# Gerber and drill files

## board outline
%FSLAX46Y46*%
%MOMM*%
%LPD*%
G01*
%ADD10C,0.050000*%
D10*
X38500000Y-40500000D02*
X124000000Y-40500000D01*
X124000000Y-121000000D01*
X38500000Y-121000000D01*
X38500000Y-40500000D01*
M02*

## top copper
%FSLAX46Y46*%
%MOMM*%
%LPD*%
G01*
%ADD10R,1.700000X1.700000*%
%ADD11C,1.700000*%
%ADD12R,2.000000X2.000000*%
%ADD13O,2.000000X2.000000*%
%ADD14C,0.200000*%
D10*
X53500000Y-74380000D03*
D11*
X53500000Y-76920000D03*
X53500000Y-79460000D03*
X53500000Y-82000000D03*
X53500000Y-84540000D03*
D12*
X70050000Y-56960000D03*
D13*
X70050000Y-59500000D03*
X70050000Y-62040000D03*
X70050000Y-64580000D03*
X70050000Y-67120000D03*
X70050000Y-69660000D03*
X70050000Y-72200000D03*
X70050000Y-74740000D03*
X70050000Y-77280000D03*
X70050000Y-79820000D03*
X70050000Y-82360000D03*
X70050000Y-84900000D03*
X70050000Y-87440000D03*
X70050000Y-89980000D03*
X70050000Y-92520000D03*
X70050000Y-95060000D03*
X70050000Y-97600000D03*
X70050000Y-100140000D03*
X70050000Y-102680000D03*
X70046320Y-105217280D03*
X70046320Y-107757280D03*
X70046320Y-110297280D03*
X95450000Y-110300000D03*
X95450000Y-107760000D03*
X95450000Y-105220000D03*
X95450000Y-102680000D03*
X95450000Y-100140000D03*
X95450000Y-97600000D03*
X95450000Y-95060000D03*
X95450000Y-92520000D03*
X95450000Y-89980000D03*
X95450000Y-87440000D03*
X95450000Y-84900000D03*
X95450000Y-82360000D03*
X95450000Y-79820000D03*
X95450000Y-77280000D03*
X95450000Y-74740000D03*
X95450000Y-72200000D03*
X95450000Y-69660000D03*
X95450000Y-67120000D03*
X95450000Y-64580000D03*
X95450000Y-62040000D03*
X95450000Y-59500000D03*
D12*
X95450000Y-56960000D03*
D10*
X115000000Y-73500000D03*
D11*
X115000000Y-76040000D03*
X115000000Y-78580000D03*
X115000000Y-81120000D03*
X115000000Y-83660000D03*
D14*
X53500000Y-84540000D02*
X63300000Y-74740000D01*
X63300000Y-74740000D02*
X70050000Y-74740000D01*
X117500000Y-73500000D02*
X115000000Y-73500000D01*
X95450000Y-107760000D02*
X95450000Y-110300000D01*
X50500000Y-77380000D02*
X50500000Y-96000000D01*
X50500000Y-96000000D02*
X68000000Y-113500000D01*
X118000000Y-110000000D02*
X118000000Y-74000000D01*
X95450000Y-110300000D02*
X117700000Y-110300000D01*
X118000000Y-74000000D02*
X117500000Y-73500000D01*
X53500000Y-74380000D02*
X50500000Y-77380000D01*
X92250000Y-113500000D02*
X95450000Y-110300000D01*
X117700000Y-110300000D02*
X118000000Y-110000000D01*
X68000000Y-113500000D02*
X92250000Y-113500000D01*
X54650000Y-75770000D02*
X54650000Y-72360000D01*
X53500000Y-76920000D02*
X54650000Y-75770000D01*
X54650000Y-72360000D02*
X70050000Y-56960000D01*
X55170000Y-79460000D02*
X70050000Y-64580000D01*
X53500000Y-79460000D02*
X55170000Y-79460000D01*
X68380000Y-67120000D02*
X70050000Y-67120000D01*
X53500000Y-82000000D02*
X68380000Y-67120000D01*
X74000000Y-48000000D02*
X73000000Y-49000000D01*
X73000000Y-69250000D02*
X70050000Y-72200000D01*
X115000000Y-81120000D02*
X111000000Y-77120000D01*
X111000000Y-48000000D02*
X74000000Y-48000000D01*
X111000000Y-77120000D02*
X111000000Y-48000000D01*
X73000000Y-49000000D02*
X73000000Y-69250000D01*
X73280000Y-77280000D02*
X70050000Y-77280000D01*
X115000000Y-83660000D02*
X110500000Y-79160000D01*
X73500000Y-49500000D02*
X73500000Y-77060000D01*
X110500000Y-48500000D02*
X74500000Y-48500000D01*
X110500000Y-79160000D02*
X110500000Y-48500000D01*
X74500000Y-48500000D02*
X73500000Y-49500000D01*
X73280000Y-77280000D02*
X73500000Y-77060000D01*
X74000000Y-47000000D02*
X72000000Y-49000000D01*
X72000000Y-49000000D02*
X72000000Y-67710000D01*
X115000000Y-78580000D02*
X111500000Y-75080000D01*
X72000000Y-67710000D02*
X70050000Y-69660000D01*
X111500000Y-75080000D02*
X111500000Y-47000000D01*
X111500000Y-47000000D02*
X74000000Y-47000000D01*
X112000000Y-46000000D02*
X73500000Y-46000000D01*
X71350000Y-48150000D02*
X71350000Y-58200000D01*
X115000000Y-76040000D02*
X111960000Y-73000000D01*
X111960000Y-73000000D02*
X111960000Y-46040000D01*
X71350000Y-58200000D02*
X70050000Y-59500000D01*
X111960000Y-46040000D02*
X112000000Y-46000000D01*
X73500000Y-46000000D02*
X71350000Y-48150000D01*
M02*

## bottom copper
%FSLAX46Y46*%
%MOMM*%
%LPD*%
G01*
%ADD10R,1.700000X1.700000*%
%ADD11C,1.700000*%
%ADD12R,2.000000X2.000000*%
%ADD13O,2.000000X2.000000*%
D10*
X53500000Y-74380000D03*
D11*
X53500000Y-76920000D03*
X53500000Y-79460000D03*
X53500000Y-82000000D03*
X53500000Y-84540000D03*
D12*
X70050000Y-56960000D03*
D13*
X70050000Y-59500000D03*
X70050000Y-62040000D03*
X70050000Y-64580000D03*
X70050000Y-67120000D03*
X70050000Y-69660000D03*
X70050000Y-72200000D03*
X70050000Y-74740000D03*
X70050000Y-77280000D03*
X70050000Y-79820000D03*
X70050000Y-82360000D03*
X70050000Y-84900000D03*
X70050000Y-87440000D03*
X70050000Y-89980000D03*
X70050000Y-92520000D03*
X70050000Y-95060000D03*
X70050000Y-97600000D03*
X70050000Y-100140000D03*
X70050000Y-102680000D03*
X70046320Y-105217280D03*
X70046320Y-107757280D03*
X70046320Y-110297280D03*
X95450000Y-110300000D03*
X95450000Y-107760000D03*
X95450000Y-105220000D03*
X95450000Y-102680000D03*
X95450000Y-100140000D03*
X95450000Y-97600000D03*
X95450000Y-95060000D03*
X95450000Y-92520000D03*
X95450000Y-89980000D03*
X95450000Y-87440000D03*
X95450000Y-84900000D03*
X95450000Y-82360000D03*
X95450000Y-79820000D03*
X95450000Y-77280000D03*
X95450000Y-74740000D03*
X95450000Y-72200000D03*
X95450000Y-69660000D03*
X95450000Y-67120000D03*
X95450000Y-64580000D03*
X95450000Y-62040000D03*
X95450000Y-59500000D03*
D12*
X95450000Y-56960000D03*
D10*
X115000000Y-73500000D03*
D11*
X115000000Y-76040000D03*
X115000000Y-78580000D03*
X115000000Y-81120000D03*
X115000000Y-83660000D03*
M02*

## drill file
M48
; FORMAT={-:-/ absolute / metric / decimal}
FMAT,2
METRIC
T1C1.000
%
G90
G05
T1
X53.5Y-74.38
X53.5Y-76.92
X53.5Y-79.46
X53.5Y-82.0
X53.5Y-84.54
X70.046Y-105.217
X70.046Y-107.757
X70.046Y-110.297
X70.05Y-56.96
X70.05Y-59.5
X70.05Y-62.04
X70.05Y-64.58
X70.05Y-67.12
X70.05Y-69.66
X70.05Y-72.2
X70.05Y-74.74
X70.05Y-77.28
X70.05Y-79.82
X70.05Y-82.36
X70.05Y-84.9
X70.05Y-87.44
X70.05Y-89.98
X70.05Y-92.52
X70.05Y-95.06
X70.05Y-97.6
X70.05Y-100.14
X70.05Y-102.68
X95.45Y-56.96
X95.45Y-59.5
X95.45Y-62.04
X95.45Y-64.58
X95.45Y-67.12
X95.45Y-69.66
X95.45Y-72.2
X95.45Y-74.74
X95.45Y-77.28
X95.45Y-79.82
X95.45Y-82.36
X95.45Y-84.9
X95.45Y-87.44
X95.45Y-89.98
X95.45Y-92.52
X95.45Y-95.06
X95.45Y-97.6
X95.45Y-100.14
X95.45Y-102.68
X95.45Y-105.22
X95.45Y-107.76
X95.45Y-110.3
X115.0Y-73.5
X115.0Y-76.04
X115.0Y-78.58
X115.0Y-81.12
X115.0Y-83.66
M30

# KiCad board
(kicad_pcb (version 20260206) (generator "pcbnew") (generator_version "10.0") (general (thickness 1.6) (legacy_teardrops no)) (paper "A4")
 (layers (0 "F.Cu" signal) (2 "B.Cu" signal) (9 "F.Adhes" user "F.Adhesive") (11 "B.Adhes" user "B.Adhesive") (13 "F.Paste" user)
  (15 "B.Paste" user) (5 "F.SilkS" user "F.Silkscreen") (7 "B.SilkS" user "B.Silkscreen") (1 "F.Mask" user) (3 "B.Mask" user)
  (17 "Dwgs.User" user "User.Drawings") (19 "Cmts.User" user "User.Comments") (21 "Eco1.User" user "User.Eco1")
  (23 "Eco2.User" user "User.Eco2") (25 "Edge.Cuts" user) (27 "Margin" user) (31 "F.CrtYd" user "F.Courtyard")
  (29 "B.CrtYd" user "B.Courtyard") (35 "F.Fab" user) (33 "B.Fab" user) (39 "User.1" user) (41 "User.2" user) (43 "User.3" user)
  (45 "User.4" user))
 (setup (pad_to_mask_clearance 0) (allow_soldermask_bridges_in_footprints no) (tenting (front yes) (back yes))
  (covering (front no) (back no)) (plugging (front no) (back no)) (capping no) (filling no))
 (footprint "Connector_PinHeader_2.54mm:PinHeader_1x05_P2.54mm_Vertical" (layer "F.Cu") (at 53.5 74.38)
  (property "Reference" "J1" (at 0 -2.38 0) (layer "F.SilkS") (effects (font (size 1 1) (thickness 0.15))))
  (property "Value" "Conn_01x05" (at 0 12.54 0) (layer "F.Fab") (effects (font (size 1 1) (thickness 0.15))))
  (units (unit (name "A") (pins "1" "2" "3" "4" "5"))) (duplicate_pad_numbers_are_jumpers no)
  (pad "1" thru_hole rect (at 0 0) (size 1.7 1.7) (drill 1) (layers "*.Cu" "*.Mask") (remove_unused_layers no) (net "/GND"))
  (pad "2" thru_hole circle (at 0 2.54) (size 1.7 1.7) (drill 1) (layers "*.Cu" "*.Mask") (remove_unused_layers no) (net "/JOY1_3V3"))
  (pad "3" thru_hole circle (at 0 5.08) (size 1.7 1.7) (drill 1) (layers "*.Cu" "*.Mask") (remove_unused_layers no) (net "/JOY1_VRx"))
  (pad "4" thru_hole circle (at 0 7.62) (size 1.7 1.7) (drill 1) (layers "*.Cu" "*.Mask") (remove_unused_layers no) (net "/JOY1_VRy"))
  (pad "5" thru_hole circle (at 0 10.16) (size 1.7 1.7) (drill 1) (layers "*.Cu" "*.Mask") (remove_unused_layers no) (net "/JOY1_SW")))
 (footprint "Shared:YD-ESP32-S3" (layer "F.Cu") (at 68.75 55.05)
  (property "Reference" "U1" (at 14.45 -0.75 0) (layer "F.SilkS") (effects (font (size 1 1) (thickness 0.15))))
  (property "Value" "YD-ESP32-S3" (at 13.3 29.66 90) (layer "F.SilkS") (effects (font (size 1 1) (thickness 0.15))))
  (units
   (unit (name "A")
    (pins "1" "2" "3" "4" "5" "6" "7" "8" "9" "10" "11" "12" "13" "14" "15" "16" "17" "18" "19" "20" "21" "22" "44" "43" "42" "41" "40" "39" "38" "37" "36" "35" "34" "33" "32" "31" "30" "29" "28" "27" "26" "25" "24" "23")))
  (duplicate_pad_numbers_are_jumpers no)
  (pad "1" thru_hole rect (at 1.3 1.91 270) (size 2 2) (drill 1) (layers "*.Cu" "*.Mask") (remove_unused_layers no) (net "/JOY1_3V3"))
  (pad "2" thru_hole oval (at 1.3 4.45 270) (size 2 2) (drill 1) (layers "*.Cu" "*.Mask") (remove_unused_layers no) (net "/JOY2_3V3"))
  (pad "3" thru_hole oval (at 1.3 6.99 270) (size 2 2) (drill 1) (layers "*.Cu" "*.Mask") (remove_unused_layers no)
   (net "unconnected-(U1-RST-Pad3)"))
  (pad "4" thru_hole oval (at 1.3 9.53 270) (size 2 2) (drill 1) (layers "*.Cu" "*.Mask") (remove_unused_layers no) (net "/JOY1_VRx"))
  (pad "5" thru_hole oval (at 1.3 12.07 270) (size 2 2) (drill 1) (layers "*.Cu" "*.Mask") (remove_unused_layers no) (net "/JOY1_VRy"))
  (pad "6" thru_hole oval (at 1.3 14.61 270) (size 2 2) (drill 1) (layers "*.Cu" "*.Mask") (remove_unused_layers no) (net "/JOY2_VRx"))
  (pad "7" thru_hole oval (at 1.3 17.15 270) (size 2 2) (drill 1) (layers "*.Cu" "*.Mask") (remove_unused_layers no) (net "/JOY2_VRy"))
  (pad "8" thru_hole oval (at 1.3 19.69 270) (size 2 2) (drill 1) (layers "*.Cu" "*.Mask") (remove_unused_layers no) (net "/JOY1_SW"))
  (pad "9" thru_hole oval (at 1.3 22.23 270) (size 2 2) (drill 1) (layers "*.Cu" "*.Mask") (remove_unused_layers no) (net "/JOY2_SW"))
  (pad "10" thru_hole oval (at 1.3 24.77 270) (size 2 2) (drill 1) (layers "*.Cu" "*.Mask") (remove_unused_layers no)
   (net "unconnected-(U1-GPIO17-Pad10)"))
  (pad "11" thru_hole oval (at 1.3 27.31 270) (size 2 2) (drill 1) (layers "*.Cu" "*.Mask") (remove_unused_layers no)
   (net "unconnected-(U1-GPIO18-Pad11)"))
  (pad "12" thru_hole oval (at 1.3 29.85 270) (size 2 2) (drill 1) (layers "*.Cu" "*.Mask") (remove_unused_layers no)
   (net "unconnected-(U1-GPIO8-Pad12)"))
  (pad "13" thru_hole oval (at 1.3 32.39 270) (size 2 2) (drill 1) (layers "*.Cu" "*.Mask") (remove_unused_layers no)
   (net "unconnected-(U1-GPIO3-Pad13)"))
  (pad "14" thru_hole oval (at 1.3 34.93 270) (size 2 2) (drill 1) (layers "*.Cu" "*.Mask") (remove_unused_layers no)
   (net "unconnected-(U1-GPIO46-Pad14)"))
  (pad "15" thru_hole oval (at 1.3 37.47 270) (size 2 2) (drill 1) (layers "*.Cu" "*.Mask") (remove_unused_layers no)
   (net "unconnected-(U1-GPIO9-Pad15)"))
  (pad "16" thru_hole oval (at 1.3 40.01 270) (size 2 2) (drill 1) (layers "*.Cu" "*.Mask") (remove_unused_layers no)
   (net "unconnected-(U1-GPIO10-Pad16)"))
  (pad "17" thru_hole oval (at 1.3 42.55 270) (size 2 2) (drill 1) (layers "*.Cu" "*.Mask") (remove_unused_layers no)
   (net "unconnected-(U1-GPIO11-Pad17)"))
  (pad "18" thru_hole oval (at 1.3 45.09 270) (size 2 2) (drill 1) (layers "*.Cu" "*.Mask") (remove_unused_layers no)
   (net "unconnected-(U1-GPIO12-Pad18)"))
  (pad "19" thru_hole oval (at 1.3 47.63 270) (size 2 2) (drill 1) (layers "*.Cu" "*.Mask") (remove_unused_layers no)
   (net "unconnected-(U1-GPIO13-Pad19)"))
  (pad "20" thru_hole oval (at 1.29632 50.16728 270) (size 2 2) (drill 1) (layers "*.Cu" "*.Mask") (remove_unused_layers no)
   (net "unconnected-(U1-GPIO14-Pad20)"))
  (pad "21" thru_hole oval (at 1.29632 52.70728 270) (size 2 2) (drill 1) (layers "*.Cu" "*.Mask") (remove_unused_layers no)
   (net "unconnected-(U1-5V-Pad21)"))
  (pad "22" thru_hole oval (at 1.29632 55.24728 270) (size 2 2) (drill 1) (layers "*.Cu" "*.Mask") (remove_unused_layers no)
   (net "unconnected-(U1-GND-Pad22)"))
  (pad "23" thru_hole oval (at 26.7 55.25 270) (size 2 2) (drill 1) (layers "*.Cu" "*.Mask") (remove_unused_layers no) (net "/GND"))
  (pad "24" thru_hole oval (at 26.7 52.71 270) (size 2 2) (drill 1) (layers "*.Cu" "*.Mask") (remove_unused_layers no) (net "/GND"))
  (pad "25" thru_hole oval (at 26.7 50.17 270) (size 2 2) (drill 1) (layers "*.Cu" "*.Mask") (remove_unused_layers no)
   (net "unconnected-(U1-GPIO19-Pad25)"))
  (pad "26" thru_hole oval (at 26.7 47.63 270) (size 2 2) (drill 1) (layers "*.Cu" "*.Mask") (remove_unused_layers no)
   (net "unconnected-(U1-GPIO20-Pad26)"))
  (pad "27" thru_hole oval (at 26.7 45.09 270) (size 2 2) (drill 1) (layers "*.Cu" "*.Mask") (remove_unused_layers no)
   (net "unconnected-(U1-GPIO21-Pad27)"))
  (pad "28" thru_hole oval (at 26.7 42.55 270) (size 2 2) (drill 1) (layers "*.Cu" "*.Mask") (remove_unused_layers no)
   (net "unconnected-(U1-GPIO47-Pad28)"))
  (pad "29" thru_hole oval (at 26.7 40.01 270) (size 2 2) (drill 1) (layers "*.Cu" "*.Mask") (remove_unused_layers no)
   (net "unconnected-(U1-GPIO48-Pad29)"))
  (pad "30" thru_hole oval (at 26.7 37.47 270) (size 2 2) (drill 1) (layers "*.Cu" "*.Mask") (remove_unused_layers no)
   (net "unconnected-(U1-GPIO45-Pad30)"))
  (pad "31" thru_hole oval (at 26.7 34.93 270) (size 2 2) (drill 1) (layers "*.Cu" "*.Mask") (remove_unused_layers no)
   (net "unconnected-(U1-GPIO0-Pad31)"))
  (pad "32" thru_hole oval (at 26.7 32.39 270) (size 2 2) (drill 1) (layers "*.Cu" "*.Mask") (remove_unused_layers no)
   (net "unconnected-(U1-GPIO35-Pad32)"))
  (pad "33" thru_hole oval (at 26.7 29.85 270) (size 2 2) (drill 1) (layers "*.Cu" "*.Mask") (remove_unused_layers no)
   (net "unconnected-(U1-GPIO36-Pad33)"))
  (pad "34" thru_hole oval (at 26.7 27.31 270) (size 2 2) (drill 1) (layers "*.Cu" "*.Mask") (remove_unused_layers no)
   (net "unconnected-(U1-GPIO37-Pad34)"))
  (pad "35" thru_hole oval (at 26.7 24.77 270) (size 2 2) (drill 1) (layers "*.Cu" "*.Mask") (remove_unused_layers no)
   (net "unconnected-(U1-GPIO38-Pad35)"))
  (pad "36" thru_hole oval (at 26.7 22.23 270) (size 2 2) (drill 1) (layers "*.Cu" "*.Mask") (remove_unused_layers no)
   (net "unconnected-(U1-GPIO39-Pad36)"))
  (pad "37" thru_hole oval (at 26.7 19.69 270) (size 2 2) (drill 1) (layers "*.Cu" "*.Mask") (remove_unused_layers no)
   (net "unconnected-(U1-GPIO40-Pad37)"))
  (pad "38" thru_hole oval (at 26.7 17.15 270) (size 2 2) (drill 1) (layers "*.Cu" "*.Mask") (remove_unused_layers no)
   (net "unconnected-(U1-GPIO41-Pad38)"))
  (pad "39" thru_hole oval (at 26.7 14.61 270) (size 2 2) (drill 1) (layers "*.Cu" "*.Mask") (remove_unused_layers no)
   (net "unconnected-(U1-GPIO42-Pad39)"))
  (pad "40" thru_hole oval (at 26.7 12.07 270) (size 2 2) (drill 1) (layers "*.Cu" "*.Mask") (remove_unused_layers no)
   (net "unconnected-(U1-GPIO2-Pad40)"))
  (pad "41" thru_hole oval (at 26.7 9.53 270) (size 2 2) (drill 1) (layers "*.Cu" "*.Mask") (remove_unused_layers no)
   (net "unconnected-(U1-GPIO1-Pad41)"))
  (pad "42" thru_hole oval (at 26.7 6.99 270) (size 2 2) (drill 1) (layers "*.Cu" "*.Mask") (remove_unused_layers no)
   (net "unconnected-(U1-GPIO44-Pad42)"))
  (pad "43" thru_hole oval (at 26.7 4.45 270) (size 2 2) (drill 1) (layers "*.Cu" "*.Mask") (remove_unused_layers no)
   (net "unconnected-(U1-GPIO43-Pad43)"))
  (pad "44" thru_hole rect (at 26.7 1.91 270) (size 2 2) (drill 1) (layers "*.Cu" "*.Mask") (remove_unused_layers no)
   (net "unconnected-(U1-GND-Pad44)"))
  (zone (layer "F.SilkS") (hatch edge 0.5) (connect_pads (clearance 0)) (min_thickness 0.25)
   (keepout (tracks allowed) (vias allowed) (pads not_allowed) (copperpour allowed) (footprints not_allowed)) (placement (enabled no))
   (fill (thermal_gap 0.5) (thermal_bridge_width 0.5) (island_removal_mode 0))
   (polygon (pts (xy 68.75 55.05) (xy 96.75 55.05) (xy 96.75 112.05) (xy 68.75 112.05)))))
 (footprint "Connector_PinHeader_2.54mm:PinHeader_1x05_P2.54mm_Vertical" (layer "F.Cu") (at 115 73.5)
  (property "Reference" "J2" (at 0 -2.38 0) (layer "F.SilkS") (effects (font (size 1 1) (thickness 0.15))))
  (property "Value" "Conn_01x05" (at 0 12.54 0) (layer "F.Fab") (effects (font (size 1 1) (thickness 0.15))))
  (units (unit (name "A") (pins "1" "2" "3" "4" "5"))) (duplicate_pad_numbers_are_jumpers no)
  (pad "1" thru_hole rect (at 0 0) (size 1.7 1.7) (drill 1) (layers "*.Cu" "*.Mask") (remove_unused_layers no) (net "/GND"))
  (pad "2" thru_hole circle (at 0 2.54) (size 1.7 1.7) (drill 1) (layers "*.Cu" "*.Mask") (remove_unused_layers no) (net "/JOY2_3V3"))
  (pad "3" thru_hole circle (at 0 5.08) (size 1.7 1.7) (drill 1) (layers "*.Cu" "*.Mask") (remove_unused_layers no) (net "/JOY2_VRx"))
  (pad "4" thru_hole circle (at 0 7.62) (size 1.7 1.7) (drill 1) (layers "*.Cu" "*.Mask") (remove_unused_layers no) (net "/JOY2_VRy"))
  (pad "5" thru_hole circle (at 0 10.16) (size 1.7 1.7) (drill 1) (layers "*.Cu" "*.Mask") (remove_unused_layers no) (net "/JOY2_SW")))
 (gr_rect (start 38.5 40.5) (end 124 121) (stroke (width 0.05) (type default)) (fill no) (layer "Edge.Cuts"))
 (segment (start 53.5 84.54) (end 63.3 74.74) (width 0.2) (layer "F.Cu") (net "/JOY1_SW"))
 (segment (start 63.3 74.74) (end 70.05 74.74) (width 0.2) (layer "F.Cu") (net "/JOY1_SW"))
 (segment (start 117.5 73.5) (end 115 73.5) (width 0.2) (layer "F.Cu") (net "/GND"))
 (segment (start 95.45 107.76) (end 95.45 110.3) (width 0.2) (layer "F.Cu") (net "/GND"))
 (segment (start 50.5 77.38) (end 50.5 96) (width 0.2) (layer "F.Cu") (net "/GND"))
 (segment (start 50.5 96) (end 68 113.5) (width 0.2) (layer "F.Cu") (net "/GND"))
 (segment (start 118 110) (end 118 74) (width 0.2) (layer "F.Cu") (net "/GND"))
 (segment (start 95.45 110.3) (end 117.7 110.3) (width 0.2) (layer "F.Cu") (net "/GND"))
 (segment (start 118 74) (end 117.5 73.5) (width 0.2) (layer "F.Cu") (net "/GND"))
 (segment (start 53.5 74.38) (end 50.5 77.38) (width 0.2) (layer "F.Cu") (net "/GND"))
 (segment (start 92.25 113.5) (end 95.45 110.3) (width 0.2) (layer "F.Cu") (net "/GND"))
 (segment (start 117.7 110.3) (end 118 110) (width 0.2) (layer "F.Cu") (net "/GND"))
 (segment (start 68 113.5) (end 92.25 113.5) (width 0.2) (layer "F.Cu") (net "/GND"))
 (segment (start 54.65 75.77) (end 54.65 72.36) (width 0.2) (layer "F.Cu") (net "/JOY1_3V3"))
 (segment (start 53.5 76.92) (end 54.65 75.77) (width 0.2) (layer "F.Cu") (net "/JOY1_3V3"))
 (segment (start 54.65 72.36) (end 70.05 56.96) (width 0.2) (layer "F.Cu") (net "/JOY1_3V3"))
 (segment (start 55.17 79.46) (end 70.05 64.58) (width 0.2) (layer "F.Cu") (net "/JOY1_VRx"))
 (segment (start 53.5 79.46) (end 55.17 79.46) (width 0.2) (layer "F.Cu") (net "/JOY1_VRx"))
 (segment (start 68.38 67.12) (end 70.05 67.12) (width 0.2) (layer "F.Cu") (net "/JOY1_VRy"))
 (segment (start 53.5 82) (end 68.38 67.12) (width 0.2) (layer "F.Cu") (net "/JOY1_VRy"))
 (segment (start 74 48) (end 73 49) (width 0.2) (layer "F.Cu") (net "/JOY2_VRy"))
 (segment (start 73 69.25) (end 70.05 72.2) (width 0.2) (layer "F.Cu") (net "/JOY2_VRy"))
 (segment (start 115 81.12) (end 111 77.12) (width 0.2) (layer "F.Cu") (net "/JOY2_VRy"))
 (segment (start 111 48) (end 74 48) (width 0.2) (layer "F.Cu") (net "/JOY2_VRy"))
 (segment (start 111 77.12) (end 111 48) (width 0.2) (layer "F.Cu") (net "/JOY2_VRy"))
 (segment (start 73 49) (end 73 69.25) (width 0.2) (layer "F.Cu") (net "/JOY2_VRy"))
 (segment (start 73.28 77.28) (end 70.05 77.28) (width 0.2) (layer "F.Cu") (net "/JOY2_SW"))
 (segment (start 115 83.66) (end 110.5 79.16) (width 0.2) (layer "F.Cu") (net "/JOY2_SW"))
 (segment (start 73.5 49.5) (end 73.5 77.06) (width 0.2) (layer "F.Cu") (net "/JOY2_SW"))
 (segment (start 110.5 48.5) (end 74.5 48.5) (width 0.2) (layer "F.Cu") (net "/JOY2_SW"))
 (segment (start 110.5 79.16) (end 110.5 48.5) (width 0.2) (layer "F.Cu") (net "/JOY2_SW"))
 (segment (start 74.5 48.5) (end 73.5 49.5) (width 0.2) (layer "F.Cu") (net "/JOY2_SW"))
 (segment (start 73.28 77.28) (end 73.5 77.06) (width 0.2) (layer "F.Cu") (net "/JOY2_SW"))
 (segment (start 74 47) (end 72 49) (width 0.2) (layer "F.Cu") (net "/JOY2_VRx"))
 (segment (start 72 49) (end 72 67.71) (width 0.2) (layer "F.Cu") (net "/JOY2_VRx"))
 (segment (start 115 78.58) (end 111.5 75.08) (width 0.2) (layer "F.Cu") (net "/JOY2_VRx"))
 (segment (start 72 67.71) (end 70.05 69.66) (width 0.2) (layer "F.Cu") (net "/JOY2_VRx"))
 (segment (start 111.5 75.08) (end 111.5 47) (width 0.2) (layer "F.Cu") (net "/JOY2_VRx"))
 (segment (start 111.5 47) (end 74 47) (width 0.2) (layer "F.Cu") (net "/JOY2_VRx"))
 (segment (start 112 46) (end 73.5 46) (width 0.2) (layer "F.Cu") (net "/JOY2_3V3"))
 (segment (start 71.35 48.15) (end 71.35 58.2) (width 0.2) (layer "F.Cu") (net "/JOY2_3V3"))
 (segment (start 115 76.04) (end 111.96 73) (width 0.2) (layer "F.Cu") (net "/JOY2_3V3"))
 (segment (start 111.96 73) (end 111.96 46.04) (width 0.2) (layer "F.Cu") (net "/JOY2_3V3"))
 (segment (start 71.35 58.2) (end 70.05 59.5) (width 0.2) (layer "F.Cu") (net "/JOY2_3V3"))
 (segment (start 111.96 46.04) (end 112 46) (width 0.2) (layer "F.Cu") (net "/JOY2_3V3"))
 (segment (start 73.5 46) (end 71.35 48.15) (width 0.2) (layer "F.Cu") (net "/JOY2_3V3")))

